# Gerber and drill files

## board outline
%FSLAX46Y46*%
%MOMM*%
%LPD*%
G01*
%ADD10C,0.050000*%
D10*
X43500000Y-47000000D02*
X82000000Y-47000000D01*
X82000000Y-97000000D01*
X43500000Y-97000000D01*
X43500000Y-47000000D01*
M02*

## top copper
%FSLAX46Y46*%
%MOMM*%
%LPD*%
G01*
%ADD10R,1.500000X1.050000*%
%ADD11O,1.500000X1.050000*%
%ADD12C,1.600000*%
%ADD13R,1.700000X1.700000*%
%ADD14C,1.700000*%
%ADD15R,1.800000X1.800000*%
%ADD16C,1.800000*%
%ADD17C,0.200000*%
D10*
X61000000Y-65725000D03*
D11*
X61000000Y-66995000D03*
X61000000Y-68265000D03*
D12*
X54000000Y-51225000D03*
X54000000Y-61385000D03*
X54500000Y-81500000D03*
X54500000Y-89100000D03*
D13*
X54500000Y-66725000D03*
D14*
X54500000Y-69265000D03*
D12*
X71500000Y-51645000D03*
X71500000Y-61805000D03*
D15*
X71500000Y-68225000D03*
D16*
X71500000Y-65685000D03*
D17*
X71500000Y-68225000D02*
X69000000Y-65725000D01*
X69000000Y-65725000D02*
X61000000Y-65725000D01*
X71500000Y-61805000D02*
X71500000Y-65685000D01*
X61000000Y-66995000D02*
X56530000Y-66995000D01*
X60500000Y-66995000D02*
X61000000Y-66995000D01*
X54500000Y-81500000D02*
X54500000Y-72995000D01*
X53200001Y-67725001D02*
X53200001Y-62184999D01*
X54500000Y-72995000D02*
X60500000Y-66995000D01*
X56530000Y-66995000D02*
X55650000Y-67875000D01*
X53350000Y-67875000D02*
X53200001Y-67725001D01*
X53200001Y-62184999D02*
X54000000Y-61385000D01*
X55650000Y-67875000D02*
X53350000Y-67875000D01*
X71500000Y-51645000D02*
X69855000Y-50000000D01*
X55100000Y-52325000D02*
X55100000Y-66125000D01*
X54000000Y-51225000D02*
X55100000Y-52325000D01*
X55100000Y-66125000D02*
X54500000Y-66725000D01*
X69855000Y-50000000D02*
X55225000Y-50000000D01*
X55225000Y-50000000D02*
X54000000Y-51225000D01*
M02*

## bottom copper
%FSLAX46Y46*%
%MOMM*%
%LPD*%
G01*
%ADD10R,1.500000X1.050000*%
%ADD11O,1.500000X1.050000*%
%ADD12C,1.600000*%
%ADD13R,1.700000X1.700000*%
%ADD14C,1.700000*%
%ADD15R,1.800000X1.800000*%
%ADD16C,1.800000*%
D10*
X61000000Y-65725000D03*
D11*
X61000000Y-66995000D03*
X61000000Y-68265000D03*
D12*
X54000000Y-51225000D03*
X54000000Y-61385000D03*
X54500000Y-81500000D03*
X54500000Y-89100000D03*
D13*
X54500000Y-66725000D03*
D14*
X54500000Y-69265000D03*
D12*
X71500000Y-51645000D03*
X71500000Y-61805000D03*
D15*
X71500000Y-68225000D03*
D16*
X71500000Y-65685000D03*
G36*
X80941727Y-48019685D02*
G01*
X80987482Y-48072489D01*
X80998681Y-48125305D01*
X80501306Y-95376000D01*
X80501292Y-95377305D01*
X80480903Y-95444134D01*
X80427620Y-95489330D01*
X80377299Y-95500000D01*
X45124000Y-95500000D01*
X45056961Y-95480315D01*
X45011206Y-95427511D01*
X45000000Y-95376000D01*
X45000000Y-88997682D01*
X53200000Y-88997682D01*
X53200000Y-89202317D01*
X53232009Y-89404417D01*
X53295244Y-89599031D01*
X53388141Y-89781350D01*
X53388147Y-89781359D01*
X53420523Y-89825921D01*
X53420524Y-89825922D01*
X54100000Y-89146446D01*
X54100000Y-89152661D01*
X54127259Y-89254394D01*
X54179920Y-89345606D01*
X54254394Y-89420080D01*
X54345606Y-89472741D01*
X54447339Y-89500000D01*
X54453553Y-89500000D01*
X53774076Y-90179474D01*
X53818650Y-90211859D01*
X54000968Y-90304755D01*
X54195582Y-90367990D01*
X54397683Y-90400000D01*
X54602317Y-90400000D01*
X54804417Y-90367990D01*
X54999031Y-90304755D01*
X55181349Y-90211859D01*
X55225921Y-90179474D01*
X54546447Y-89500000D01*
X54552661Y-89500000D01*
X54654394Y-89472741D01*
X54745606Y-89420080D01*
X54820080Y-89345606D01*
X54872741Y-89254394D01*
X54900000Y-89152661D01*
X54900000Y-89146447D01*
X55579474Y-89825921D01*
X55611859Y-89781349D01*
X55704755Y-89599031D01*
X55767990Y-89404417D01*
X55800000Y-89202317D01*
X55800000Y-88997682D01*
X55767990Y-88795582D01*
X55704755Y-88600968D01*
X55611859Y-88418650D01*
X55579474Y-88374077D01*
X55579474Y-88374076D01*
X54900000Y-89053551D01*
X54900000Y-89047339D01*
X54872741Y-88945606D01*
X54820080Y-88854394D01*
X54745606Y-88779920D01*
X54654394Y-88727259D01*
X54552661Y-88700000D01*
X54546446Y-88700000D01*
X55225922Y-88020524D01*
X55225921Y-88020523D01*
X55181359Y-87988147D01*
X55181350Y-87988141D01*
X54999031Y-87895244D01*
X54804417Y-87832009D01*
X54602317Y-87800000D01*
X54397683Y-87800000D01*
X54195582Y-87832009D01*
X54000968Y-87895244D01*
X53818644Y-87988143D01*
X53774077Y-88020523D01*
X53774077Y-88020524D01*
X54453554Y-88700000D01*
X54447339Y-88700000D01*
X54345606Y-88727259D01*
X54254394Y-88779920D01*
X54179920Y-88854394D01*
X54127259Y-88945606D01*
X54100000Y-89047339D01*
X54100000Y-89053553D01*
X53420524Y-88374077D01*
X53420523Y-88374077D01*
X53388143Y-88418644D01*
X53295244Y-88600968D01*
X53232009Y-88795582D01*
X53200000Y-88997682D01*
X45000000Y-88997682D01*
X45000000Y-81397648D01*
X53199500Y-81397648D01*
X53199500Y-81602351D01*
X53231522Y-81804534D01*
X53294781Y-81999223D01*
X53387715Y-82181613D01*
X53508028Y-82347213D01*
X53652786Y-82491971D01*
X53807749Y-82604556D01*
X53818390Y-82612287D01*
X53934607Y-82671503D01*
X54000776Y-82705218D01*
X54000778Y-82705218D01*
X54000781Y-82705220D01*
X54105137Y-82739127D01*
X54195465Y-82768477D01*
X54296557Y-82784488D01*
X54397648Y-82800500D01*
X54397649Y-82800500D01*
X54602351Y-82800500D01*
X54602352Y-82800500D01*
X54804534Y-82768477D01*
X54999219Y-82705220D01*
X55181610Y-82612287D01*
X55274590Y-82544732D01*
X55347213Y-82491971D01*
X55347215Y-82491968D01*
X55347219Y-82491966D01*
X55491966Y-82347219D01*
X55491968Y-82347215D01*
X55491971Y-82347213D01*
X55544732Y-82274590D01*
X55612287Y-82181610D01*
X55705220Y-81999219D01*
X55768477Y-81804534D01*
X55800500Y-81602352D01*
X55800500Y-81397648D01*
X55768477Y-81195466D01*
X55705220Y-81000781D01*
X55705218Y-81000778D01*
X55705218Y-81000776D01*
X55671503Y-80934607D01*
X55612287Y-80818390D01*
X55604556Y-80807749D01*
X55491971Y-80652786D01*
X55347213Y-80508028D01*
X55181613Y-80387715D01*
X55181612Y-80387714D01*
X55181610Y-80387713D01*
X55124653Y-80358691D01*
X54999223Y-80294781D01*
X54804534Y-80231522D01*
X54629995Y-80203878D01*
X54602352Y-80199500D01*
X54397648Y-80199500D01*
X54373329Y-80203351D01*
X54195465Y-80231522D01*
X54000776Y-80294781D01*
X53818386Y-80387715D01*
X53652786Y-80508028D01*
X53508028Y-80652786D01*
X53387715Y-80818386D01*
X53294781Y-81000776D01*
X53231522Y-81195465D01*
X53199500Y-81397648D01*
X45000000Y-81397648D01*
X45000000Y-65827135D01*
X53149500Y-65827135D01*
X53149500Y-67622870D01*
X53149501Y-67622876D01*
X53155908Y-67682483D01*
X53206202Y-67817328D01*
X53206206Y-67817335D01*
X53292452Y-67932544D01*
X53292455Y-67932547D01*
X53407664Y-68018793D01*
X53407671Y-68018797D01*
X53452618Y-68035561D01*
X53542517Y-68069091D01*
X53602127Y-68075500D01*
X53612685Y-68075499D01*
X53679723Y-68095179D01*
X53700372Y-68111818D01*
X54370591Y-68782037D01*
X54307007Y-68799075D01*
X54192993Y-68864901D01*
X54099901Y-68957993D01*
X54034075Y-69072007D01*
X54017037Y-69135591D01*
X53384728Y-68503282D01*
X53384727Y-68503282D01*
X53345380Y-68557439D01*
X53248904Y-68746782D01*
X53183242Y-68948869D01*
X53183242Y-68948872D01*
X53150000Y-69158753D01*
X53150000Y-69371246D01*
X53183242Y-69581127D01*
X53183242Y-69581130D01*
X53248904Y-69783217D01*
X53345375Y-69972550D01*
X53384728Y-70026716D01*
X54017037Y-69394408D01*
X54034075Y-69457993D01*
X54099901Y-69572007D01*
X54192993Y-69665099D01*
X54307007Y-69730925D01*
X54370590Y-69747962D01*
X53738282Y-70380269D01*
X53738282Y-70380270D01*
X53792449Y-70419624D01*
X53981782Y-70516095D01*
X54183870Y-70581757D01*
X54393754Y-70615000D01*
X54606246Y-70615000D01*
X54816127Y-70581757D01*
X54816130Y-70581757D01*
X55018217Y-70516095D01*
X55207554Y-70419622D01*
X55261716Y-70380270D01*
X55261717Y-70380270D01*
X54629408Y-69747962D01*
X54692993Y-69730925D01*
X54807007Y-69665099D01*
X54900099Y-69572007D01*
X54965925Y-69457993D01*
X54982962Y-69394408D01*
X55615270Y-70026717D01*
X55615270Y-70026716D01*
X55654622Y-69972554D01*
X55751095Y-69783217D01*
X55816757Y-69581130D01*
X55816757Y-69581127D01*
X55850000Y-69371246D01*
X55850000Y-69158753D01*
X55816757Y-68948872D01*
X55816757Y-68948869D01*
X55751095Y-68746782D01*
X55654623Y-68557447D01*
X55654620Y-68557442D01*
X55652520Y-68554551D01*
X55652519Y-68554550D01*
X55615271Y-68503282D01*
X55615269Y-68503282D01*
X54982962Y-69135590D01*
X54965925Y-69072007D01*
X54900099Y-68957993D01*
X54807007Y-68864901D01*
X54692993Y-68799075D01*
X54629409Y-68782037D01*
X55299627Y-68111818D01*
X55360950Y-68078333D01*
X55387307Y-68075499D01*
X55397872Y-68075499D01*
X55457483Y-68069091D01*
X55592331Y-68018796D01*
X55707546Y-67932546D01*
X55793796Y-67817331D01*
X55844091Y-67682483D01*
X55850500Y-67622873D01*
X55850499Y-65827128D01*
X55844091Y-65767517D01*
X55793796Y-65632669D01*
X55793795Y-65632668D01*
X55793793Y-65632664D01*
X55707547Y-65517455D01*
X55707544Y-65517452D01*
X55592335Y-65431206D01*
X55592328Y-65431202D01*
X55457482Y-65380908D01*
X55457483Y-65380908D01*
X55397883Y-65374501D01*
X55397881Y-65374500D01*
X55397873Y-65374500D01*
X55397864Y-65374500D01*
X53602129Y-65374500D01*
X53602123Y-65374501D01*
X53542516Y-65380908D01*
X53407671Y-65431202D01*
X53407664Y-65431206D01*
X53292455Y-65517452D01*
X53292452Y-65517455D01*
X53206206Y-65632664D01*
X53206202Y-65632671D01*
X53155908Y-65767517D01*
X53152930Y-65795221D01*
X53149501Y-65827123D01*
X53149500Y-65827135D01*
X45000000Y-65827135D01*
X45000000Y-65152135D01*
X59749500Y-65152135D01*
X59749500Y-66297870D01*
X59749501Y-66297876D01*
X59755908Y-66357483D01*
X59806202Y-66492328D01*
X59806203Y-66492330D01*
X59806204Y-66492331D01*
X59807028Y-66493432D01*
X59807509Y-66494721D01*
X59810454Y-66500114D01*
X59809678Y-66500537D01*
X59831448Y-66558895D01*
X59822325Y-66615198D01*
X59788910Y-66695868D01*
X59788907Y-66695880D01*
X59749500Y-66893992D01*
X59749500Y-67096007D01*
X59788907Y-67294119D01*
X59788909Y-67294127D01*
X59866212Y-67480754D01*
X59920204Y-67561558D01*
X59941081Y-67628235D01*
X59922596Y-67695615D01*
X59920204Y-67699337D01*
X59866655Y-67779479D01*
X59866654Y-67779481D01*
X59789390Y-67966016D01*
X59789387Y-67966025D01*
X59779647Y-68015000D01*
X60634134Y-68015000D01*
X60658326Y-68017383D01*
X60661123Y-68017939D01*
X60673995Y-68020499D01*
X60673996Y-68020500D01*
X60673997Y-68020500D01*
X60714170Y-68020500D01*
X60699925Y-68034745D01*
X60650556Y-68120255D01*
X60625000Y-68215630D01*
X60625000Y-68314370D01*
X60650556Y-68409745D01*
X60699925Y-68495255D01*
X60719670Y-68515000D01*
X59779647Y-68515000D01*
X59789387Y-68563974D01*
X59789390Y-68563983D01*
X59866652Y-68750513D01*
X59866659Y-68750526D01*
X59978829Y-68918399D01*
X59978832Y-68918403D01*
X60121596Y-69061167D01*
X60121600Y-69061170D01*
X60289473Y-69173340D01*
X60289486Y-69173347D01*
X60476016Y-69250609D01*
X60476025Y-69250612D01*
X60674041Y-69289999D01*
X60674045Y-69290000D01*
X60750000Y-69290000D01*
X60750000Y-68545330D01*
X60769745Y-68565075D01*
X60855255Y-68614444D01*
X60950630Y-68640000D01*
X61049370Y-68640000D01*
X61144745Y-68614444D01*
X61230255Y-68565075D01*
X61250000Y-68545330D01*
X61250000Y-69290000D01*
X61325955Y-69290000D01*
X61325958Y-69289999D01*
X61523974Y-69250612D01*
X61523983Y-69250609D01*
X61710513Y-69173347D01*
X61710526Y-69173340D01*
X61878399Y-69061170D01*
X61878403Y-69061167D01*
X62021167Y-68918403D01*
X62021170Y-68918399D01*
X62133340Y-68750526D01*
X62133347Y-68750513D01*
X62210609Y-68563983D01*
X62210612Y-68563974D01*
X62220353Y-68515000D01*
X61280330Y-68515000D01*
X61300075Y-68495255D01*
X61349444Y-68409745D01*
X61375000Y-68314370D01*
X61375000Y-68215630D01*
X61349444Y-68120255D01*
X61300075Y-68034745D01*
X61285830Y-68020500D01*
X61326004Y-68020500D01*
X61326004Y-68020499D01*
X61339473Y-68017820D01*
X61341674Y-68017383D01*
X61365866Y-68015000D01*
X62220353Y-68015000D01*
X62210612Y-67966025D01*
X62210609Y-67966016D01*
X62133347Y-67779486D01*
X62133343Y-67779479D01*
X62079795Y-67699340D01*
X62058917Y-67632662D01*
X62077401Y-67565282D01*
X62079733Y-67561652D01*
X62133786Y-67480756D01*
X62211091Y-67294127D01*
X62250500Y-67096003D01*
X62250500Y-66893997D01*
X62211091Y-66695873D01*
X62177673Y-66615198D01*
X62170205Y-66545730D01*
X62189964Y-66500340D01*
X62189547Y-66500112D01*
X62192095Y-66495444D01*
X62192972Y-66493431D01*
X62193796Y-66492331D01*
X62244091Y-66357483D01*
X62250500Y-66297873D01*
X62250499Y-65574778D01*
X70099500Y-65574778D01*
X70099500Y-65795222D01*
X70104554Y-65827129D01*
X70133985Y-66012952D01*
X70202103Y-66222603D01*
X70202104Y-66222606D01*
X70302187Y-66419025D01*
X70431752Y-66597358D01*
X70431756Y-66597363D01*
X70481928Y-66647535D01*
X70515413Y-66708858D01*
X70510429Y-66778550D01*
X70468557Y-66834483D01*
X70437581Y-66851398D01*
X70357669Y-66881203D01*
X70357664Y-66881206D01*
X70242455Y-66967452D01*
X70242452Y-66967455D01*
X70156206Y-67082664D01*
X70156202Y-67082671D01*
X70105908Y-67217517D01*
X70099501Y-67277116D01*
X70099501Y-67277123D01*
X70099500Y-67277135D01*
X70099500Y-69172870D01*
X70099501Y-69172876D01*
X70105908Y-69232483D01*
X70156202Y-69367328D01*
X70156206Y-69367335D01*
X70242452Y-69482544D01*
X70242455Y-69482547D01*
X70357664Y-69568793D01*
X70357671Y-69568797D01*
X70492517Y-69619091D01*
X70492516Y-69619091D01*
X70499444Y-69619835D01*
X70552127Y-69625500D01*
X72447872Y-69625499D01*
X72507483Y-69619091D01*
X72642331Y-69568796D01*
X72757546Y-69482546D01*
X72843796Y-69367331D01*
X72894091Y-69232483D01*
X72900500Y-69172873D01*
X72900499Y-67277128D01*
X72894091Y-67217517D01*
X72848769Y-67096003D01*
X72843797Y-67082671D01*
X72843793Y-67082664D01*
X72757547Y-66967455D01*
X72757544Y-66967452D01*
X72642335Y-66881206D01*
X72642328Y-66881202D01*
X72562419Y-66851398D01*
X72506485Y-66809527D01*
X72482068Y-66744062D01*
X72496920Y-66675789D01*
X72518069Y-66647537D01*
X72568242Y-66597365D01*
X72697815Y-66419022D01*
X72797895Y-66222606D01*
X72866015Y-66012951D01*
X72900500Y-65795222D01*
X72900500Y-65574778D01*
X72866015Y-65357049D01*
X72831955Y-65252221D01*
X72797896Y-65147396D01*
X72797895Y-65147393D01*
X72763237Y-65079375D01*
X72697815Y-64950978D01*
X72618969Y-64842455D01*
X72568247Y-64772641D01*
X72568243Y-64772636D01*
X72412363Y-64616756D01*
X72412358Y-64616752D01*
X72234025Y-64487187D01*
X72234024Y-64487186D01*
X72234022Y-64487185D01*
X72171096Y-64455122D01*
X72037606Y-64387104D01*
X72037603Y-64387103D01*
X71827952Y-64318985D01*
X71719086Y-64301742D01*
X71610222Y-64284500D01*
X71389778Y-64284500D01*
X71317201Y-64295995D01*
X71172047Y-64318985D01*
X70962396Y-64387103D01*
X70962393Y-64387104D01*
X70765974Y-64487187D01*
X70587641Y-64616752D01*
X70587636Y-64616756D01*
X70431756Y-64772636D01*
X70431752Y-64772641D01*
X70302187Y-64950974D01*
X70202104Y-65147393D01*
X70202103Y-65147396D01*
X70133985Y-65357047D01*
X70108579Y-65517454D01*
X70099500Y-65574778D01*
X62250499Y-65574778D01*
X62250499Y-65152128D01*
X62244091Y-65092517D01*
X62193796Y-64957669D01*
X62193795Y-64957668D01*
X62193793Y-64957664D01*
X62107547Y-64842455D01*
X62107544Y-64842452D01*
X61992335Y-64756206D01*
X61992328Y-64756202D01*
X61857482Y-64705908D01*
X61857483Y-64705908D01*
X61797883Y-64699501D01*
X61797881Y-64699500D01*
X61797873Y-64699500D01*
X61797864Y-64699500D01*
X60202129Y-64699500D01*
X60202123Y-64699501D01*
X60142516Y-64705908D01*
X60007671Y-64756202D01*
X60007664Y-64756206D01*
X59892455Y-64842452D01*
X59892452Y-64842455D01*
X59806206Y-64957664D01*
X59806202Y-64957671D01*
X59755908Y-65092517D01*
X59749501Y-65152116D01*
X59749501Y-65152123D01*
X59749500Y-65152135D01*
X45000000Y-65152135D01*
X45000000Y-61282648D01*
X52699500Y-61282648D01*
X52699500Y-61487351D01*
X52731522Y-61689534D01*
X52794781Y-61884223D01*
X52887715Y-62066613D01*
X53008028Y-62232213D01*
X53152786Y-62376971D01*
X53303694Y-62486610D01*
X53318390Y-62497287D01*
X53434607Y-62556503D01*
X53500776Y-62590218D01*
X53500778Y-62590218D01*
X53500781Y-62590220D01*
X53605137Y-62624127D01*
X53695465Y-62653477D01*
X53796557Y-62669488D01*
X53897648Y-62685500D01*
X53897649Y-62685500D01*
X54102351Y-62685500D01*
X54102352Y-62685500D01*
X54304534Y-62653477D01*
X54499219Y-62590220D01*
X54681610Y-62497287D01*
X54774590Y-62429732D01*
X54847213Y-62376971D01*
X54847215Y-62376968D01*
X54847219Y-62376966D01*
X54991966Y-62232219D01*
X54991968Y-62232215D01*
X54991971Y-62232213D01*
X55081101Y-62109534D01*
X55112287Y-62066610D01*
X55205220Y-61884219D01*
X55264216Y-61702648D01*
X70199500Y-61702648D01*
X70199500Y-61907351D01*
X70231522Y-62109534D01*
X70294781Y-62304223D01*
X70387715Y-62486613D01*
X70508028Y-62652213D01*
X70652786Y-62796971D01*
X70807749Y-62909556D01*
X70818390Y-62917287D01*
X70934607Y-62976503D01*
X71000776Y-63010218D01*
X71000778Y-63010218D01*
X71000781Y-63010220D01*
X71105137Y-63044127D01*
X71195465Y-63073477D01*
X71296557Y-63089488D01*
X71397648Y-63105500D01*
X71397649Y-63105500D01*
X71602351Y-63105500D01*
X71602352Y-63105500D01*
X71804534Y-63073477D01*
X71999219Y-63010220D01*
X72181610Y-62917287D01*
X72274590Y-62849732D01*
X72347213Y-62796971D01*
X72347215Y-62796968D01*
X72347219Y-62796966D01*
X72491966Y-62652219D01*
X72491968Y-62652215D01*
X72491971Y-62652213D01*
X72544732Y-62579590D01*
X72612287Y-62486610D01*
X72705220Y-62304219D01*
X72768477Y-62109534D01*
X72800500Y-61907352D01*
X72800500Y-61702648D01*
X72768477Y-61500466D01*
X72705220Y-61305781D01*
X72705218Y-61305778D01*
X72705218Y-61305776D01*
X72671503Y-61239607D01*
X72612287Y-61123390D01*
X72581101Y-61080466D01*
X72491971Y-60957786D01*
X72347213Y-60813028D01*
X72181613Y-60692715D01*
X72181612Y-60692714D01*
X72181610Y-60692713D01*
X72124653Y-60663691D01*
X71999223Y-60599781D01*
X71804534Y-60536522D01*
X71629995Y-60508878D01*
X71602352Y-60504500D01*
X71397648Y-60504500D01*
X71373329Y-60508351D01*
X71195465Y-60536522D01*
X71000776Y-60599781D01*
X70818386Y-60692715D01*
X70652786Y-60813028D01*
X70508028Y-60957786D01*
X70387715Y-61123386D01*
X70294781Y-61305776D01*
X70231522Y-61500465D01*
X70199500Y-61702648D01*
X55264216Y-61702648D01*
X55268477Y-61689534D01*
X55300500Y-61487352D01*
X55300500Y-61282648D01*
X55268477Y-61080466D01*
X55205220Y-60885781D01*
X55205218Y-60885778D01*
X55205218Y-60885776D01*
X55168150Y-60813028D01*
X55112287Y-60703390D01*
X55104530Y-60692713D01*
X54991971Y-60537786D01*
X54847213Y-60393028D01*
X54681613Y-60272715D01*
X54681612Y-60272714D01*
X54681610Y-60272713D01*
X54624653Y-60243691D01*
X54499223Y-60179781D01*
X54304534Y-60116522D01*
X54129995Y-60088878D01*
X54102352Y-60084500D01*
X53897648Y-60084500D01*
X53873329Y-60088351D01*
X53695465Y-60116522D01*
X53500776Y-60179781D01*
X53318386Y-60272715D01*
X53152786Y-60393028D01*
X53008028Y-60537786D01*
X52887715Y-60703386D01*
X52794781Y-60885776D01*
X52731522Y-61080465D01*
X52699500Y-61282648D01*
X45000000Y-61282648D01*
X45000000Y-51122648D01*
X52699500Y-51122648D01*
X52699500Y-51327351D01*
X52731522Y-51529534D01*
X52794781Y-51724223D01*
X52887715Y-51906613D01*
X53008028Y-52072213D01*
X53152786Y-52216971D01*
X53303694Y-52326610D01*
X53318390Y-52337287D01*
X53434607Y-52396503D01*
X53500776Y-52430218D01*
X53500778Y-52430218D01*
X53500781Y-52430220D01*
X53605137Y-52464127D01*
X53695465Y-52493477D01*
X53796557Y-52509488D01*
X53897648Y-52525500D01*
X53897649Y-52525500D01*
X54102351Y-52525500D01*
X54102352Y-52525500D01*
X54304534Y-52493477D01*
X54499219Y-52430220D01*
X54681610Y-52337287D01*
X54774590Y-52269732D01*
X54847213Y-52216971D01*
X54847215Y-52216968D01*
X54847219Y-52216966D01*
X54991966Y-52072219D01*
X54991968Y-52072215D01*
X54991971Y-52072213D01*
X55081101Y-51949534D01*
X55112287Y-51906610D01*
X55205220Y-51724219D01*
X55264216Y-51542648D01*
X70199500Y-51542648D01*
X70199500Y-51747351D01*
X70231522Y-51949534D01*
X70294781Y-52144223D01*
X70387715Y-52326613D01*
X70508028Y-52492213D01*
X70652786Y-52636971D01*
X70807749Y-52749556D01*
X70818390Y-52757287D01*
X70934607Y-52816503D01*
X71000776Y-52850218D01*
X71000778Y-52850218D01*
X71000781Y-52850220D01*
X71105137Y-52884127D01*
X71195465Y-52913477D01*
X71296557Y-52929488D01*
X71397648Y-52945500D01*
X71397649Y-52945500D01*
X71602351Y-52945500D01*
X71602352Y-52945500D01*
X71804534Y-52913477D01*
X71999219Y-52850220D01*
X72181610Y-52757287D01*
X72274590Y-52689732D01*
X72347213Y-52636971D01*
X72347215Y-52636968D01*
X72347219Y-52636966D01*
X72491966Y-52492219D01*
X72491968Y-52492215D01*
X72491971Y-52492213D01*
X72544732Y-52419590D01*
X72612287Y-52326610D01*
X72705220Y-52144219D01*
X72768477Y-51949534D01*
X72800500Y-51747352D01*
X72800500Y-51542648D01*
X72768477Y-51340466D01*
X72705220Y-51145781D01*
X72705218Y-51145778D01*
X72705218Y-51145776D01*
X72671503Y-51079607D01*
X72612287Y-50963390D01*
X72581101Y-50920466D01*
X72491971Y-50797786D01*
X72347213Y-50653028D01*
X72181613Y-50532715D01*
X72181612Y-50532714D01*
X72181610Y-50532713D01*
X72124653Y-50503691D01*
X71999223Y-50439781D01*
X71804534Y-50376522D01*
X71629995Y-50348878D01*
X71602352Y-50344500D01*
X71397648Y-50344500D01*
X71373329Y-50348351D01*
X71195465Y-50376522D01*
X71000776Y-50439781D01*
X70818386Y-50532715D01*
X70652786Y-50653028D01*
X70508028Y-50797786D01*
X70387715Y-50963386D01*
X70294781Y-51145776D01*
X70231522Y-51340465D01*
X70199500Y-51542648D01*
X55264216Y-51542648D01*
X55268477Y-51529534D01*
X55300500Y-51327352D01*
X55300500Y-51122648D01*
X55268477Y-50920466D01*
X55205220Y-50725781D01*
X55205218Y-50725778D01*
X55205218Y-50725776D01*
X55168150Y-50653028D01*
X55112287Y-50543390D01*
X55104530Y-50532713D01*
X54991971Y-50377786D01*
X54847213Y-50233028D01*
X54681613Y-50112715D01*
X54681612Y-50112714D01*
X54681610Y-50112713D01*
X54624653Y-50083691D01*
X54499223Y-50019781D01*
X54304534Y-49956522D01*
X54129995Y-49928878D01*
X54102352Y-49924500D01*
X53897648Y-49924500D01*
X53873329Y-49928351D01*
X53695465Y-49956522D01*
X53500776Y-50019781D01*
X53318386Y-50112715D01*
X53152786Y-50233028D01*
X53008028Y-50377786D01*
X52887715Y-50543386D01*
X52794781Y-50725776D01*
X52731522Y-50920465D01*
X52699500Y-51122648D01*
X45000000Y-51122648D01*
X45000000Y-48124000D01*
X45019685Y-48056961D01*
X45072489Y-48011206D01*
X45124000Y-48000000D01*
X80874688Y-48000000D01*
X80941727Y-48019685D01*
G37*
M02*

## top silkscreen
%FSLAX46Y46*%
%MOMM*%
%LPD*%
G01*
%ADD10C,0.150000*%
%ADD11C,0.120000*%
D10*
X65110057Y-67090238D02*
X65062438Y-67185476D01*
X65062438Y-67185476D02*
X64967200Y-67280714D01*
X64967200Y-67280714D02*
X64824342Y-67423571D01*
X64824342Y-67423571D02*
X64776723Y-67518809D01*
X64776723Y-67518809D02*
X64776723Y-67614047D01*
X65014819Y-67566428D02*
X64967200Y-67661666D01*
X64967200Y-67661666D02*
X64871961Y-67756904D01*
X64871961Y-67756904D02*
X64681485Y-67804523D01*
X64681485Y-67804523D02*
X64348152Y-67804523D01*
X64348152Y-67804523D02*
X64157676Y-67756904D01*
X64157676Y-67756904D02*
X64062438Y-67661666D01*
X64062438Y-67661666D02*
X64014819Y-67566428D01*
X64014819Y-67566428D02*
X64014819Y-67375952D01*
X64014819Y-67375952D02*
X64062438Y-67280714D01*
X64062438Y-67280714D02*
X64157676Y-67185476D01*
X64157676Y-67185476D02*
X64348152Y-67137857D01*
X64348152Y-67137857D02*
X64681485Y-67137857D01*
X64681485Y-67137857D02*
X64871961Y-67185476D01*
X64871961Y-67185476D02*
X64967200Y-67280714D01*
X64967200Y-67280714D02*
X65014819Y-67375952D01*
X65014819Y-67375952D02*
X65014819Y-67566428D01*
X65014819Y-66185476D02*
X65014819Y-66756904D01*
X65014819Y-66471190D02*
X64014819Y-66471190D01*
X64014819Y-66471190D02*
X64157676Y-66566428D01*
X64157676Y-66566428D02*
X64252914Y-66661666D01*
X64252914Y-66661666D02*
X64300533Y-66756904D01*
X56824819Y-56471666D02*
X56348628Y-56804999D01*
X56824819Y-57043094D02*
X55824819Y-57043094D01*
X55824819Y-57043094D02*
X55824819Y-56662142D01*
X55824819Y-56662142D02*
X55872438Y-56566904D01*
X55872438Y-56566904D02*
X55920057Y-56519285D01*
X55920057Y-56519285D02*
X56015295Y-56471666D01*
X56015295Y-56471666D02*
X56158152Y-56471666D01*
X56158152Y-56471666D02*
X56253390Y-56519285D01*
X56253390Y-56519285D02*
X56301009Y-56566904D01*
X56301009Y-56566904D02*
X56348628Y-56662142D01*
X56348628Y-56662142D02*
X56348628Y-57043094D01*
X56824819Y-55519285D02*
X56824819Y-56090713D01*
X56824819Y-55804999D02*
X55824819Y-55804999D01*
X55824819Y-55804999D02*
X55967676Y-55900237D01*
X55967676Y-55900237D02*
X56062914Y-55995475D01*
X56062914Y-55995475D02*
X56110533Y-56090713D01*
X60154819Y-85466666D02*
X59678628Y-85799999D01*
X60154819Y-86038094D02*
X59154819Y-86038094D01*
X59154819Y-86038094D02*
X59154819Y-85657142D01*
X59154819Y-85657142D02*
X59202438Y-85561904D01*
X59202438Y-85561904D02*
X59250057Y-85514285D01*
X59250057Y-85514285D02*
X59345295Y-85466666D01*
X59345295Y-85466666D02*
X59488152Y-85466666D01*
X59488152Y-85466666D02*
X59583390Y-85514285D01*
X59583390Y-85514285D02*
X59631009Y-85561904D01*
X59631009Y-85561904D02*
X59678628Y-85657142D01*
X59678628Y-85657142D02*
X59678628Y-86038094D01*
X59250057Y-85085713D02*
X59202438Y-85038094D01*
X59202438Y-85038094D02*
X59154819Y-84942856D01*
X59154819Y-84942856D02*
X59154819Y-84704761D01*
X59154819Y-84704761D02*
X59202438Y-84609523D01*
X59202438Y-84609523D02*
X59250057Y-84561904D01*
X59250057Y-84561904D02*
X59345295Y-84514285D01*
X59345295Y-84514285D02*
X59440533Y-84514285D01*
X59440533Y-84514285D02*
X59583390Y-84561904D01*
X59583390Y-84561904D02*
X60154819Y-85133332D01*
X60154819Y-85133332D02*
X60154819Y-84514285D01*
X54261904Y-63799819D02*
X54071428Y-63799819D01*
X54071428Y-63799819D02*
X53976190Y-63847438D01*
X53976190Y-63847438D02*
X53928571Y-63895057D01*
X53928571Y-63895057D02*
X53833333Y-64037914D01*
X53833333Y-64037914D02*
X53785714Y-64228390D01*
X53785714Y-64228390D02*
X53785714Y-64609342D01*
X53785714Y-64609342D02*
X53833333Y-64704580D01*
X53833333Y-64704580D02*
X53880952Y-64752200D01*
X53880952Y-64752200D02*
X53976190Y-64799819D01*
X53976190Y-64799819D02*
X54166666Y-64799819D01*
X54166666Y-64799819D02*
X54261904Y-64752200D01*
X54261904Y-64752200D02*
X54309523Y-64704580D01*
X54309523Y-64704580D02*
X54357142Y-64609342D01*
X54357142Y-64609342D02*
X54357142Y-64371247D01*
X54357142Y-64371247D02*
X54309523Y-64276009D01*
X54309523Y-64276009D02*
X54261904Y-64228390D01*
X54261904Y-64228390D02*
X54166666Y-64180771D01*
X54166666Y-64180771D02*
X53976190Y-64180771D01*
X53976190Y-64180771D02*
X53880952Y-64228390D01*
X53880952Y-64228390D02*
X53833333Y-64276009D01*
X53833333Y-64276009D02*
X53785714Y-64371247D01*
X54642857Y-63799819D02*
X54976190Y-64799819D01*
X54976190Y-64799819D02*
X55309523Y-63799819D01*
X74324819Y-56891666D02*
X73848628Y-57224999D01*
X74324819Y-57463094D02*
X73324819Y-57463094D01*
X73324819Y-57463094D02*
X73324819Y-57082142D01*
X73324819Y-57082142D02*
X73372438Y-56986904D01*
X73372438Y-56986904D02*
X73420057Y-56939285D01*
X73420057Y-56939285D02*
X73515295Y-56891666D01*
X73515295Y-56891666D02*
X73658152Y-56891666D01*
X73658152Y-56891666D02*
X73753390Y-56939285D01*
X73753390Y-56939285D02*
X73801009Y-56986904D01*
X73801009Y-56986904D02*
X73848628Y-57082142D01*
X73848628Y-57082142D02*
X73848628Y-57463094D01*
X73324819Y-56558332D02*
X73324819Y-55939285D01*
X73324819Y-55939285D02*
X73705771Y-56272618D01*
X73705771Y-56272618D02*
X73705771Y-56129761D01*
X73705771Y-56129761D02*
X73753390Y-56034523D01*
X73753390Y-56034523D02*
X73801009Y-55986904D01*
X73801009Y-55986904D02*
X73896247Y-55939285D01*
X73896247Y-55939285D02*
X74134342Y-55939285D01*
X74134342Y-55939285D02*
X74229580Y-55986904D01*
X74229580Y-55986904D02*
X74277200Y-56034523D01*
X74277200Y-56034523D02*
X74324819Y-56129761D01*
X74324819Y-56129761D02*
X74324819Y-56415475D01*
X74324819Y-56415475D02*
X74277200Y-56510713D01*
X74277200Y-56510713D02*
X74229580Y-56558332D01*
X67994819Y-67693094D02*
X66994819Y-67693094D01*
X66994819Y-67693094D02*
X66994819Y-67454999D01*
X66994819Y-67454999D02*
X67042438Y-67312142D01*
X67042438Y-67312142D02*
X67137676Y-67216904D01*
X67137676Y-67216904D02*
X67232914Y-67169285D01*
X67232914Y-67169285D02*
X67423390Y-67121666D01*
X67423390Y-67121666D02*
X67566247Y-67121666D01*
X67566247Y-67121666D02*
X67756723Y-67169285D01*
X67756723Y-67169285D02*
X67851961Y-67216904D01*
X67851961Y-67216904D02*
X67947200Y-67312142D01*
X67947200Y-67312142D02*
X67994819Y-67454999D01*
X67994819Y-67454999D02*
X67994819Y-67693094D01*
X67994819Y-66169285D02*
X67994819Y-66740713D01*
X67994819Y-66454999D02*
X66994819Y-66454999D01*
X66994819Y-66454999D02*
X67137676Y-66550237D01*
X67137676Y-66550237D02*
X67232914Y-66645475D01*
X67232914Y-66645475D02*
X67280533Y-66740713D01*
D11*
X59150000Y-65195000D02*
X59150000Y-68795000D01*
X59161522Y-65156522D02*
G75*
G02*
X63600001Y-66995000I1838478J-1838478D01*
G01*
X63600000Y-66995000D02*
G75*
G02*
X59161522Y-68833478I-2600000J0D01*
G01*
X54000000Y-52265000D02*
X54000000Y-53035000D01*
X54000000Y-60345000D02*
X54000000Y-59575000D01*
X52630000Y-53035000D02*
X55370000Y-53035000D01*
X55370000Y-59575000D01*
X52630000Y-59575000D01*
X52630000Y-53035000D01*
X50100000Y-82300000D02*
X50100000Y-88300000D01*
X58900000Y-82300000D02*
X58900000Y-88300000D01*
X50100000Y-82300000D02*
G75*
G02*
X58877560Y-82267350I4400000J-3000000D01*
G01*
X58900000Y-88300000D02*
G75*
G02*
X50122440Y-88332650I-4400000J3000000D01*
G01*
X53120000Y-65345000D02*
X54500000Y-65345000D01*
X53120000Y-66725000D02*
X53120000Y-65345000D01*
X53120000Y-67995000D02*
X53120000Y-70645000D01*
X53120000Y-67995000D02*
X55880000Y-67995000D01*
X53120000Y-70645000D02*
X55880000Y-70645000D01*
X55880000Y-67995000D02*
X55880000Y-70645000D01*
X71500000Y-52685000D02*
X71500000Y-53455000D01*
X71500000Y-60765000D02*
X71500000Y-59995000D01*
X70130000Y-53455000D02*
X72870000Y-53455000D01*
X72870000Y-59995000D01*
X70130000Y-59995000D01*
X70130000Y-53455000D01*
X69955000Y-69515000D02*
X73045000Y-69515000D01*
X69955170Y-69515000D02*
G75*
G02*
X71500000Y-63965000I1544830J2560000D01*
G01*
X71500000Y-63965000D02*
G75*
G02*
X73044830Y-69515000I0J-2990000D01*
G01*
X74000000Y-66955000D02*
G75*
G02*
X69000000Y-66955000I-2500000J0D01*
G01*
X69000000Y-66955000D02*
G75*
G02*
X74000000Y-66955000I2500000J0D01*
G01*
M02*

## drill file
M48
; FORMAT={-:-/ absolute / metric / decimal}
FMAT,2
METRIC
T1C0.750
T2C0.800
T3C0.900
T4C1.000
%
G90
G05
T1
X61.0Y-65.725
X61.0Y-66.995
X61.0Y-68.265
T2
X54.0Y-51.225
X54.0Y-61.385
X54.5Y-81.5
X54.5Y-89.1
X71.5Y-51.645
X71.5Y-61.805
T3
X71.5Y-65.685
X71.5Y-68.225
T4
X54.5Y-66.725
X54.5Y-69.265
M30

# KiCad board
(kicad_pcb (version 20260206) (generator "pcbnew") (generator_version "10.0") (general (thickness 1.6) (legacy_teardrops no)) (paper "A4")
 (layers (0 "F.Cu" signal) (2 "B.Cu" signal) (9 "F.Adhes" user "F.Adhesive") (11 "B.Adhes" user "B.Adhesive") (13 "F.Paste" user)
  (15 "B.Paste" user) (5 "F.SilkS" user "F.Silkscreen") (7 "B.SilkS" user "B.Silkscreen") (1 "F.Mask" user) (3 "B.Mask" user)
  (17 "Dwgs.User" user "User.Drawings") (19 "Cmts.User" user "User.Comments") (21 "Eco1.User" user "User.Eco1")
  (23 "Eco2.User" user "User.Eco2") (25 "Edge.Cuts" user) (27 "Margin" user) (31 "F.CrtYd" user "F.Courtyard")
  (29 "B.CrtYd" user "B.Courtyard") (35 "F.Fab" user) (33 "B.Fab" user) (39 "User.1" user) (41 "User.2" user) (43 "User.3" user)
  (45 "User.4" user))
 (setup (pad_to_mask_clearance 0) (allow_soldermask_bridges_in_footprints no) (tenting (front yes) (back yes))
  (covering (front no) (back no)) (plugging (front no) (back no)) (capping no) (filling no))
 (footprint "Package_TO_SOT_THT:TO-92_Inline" (layer "F.Cu") (at 61 65.725 -90)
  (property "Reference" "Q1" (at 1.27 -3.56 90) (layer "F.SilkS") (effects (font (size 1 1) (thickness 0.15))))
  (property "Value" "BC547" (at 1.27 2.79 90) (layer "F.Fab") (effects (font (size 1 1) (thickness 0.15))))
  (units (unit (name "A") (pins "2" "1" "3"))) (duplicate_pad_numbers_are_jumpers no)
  (fp_line (start -0.53 1.85) (end 3.07 1.85) (stroke (width 0.12) (type solid)) (layer "F.SilkS"))
  (fp_arc (start -0.568478 1.838478) (mid -1.132087 -0.994977) (end 1.27 -2.6) (stroke (width 0.12) (type solid)) (layer "F.SilkS"))
  (fp_arc (start 1.27 -2.6) (mid 3.672087 -0.994977) (end 3.108478 1.838478) (stroke (width 0.12) (type solid)) (layer "F.SilkS"))
  (pad "1" thru_hole rect (at 0 0 270) (size 1.05 1.5) (drill 0.75) (layers "*.Cu" "*.Mask") (remove_unused_layers no) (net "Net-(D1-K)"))
  (pad "2" thru_hole oval (at 1.27 0 270) (size 1.05 1.5) (drill 0.75) (layers "*.Cu" "*.Mask") (remove_unused_layers no) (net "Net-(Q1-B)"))
  (pad "3" thru_hole oval (at 2.54 0 270) (size 1.05 1.5) (drill 0.75) (layers "*.Cu" "*.Mask") (remove_unused_layers no) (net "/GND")))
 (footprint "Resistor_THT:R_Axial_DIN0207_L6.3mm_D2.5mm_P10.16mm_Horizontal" (layer "F.Cu") (at 54 51.225 -90)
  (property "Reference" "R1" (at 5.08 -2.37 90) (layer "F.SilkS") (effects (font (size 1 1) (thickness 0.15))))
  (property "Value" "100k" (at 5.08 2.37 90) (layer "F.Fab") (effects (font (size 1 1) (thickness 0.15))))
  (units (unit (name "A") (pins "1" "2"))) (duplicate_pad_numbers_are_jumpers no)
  (fp_line (start 1.04 0) (end 1.81 0) (stroke (width 0.12) (type solid)) (layer "F.SilkS"))
  (fp_line (start 9.12 0) (end 8.35 0) (stroke (width 0.12) (type solid)) (layer "F.SilkS"))
  (fp_rect (start 1.81 -1.37) (end 8.35 1.37) (stroke (width 0.12) (type solid)) (fill no) (layer "F.SilkS"))
  (pad "1" thru_hole circle (at 0 0 270) (size 1.6 1.6) (drill 0.8) (layers "*.Cu" "*.Mask") (remove_unused_layers no) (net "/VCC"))
  (pad "2" thru_hole circle (at 10.16 0 270) (size 1.6 1.6) (drill 0.8) (layers "*.Cu" "*.Mask") (remove_unused_layers no)
   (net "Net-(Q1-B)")))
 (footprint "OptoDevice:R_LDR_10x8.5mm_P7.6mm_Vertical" (layer "F.Cu") (at 54.5 81.5 -90)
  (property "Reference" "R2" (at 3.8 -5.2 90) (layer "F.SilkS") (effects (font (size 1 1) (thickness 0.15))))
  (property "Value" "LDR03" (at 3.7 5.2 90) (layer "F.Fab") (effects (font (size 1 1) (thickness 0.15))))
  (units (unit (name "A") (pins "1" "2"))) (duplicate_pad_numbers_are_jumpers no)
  (fp_line (start 0.8 4.4) (end 6.8 4.4) (stroke (width 0.12) (type solid)) (layer "F.SilkS"))
  (fp_line (start 0.8 -4.4) (end 6.8 -4.4) (stroke (width 0.12) (type solid)) (layer "F.SilkS"))
  (fp_arc (start 0.8 4.4) (mid -1.525374 0.019809) (end 0.76735 -4.37756) (stroke (width 0.12) (type solid)) (layer "F.SilkS"))
  (fp_arc (start 6.8 -4.4) (mid 9.125374 -0.019809) (end 6.83265 4.37756) (stroke (width 0.12) (type solid)) (layer "F.SilkS"))
  (pad "1" thru_hole circle (at 0 0 270) (size 1.6 1.6) (drill 0.8) (layers "*.Cu" "*.Mask") (remove_unused_layers no) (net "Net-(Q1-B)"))
  (pad "2" thru_hole circle (at 7.6 0 270) (size 1.6 1.6) (drill 0.8) (layers "*.Cu" "*.Mask") (remove_unused_layers no) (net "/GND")))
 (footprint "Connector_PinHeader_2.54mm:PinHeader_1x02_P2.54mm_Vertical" (layer "F.Cu") (at 54.5 66.725)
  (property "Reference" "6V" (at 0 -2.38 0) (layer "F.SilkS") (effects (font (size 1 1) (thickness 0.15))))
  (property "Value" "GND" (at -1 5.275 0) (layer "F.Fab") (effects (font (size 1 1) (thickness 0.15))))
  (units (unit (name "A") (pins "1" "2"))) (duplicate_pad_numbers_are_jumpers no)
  (fp_line (start -1.38 -1.38) (end 0 -1.38) (stroke (width 0.12) (type solid)) (layer "F.SilkS"))
  (fp_line (start -1.38 0) (end -1.38 -1.38) (stroke (width 0.12) (type solid)) (layer "F.SilkS"))
  (fp_line (start -1.38 1.27) (end -1.38 3.92) (stroke (width 0.12) (type solid)) (layer "F.SilkS"))
  (fp_line (start -1.38 1.27) (end 1.38 1.27) (stroke (width 0.12) (type solid)) (layer "F.SilkS"))
  (fp_line (start -1.38 3.92) (end 1.38 3.92) (stroke (width 0.12) (type solid)) (layer "F.SilkS"))
  (fp_line (start 1.38 1.27) (end 1.38 3.92) (stroke (width 0.12) (type solid)) (layer "F.SilkS"))
  (pad "1" thru_hole rect (at 0 0) (size 1.7 1.7) (drill 1) (layers "*.Cu" "*.Mask") (remove_unused_layers no) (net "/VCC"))
  (pad "2" thru_hole circle (at 0 2.54) (size 1.7 1.7) (drill 1) (layers "*.Cu" "*.Mask") (remove_unused_layers no) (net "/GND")))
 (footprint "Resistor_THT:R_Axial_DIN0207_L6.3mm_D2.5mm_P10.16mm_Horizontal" (layer "F.Cu") (at 71.5 51.645 -90)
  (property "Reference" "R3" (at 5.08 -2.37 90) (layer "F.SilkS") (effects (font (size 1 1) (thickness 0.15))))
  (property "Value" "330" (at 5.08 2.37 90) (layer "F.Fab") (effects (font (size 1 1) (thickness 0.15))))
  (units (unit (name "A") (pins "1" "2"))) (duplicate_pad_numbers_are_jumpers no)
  (fp_line (start 1.04 0) (end 1.81 0) (stroke (width 0.12) (type solid)) (layer "F.SilkS"))
  (fp_line (start 9.12 0) (end 8.35 0) (stroke (width 0.12) (type solid)) (layer "F.SilkS"))
  (fp_rect (start 1.81 -1.37) (end 8.35 1.37) (stroke (width 0.12) (type solid)) (fill no) (layer "F.SilkS"))
  (pad "1" thru_hole circle (at 0 0 270) (size 1.6 1.6) (drill 0.8) (layers "*.Cu" "*.Mask") (remove_unused_layers no) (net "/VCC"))
  (pad "2" thru_hole circle (at 10.16 0 270) (size 1.6 1.6) (drill 0.8) (layers "*.Cu" "*.Mask") (remove_unused_layers no)
   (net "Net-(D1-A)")))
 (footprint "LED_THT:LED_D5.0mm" (layer "F.Cu") (at 71.5 68.225 90)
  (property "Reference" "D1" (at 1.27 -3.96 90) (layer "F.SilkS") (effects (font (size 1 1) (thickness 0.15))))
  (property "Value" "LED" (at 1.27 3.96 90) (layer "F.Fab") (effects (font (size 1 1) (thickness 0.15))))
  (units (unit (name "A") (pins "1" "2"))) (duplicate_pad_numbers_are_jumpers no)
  (fp_line (start -1.29 -1.545) (end -1.29 1.545) (stroke (width 0.12) (type solid)) (layer "F.SilkS"))
  (fp_arc (start -1.29 -1.54483) (mid 2.071779 -2.880495) (end 4.26 0) (stroke (width 0.12) (type solid)) (layer "F.SilkS"))
  (fp_arc (start 4.26 0) (mid 2.071779 2.880495) (end -1.29 1.54483) (stroke (width 0.12) (type solid)) (layer "F.SilkS"))
  (fp_circle (center 1.27 0) (end 3.77 0) (stroke (width 0.12) (type solid)) (fill no) (layer "F.SilkS"))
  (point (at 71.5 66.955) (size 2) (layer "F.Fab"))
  (pad "1" thru_hole rect (at 0 0 90) (size 1.8 1.8) (drill 0.9) (layers "*.Cu" "*.Mask") (remove_unused_layers no) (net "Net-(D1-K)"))
  (pad "2" thru_hole circle (at 2.54 0 90) (size 1.8 1.8) (drill 0.9) (layers "*.Cu" "*.Mask") (remove_unused_layers no) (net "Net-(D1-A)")))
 (gr_rect (start 43.5 47) (end 82 97) (stroke (width 0.05) (type default)) (fill no) (layer "Edge.Cuts"))
 (segment (start 71.5 68.225) (end 69 65.725) (width 0.2) (layer "F.Cu") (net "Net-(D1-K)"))
 (segment (start 69 65.725) (end 61 65.725) (width 0.2) (layer "F.Cu") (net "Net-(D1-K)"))
 (segment (start 71.5 61.805) (end 71.5 65.685) (width 0.2) (layer "F.Cu") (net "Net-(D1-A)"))
 (segment (start 61 66.995) (end 56.53 66.995) (width 0.2) (layer "F.Cu") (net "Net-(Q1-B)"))
 (segment (start 60.5 66.995) (end 61 66.995) (width 0.2) (layer "F.Cu") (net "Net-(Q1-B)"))
 (segment (start 54.5 81.5) (end 54.5 72.995) (width 0.2) (layer "F.Cu") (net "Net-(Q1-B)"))
 (segment (start 53.200001 67.725001) (end 53.200001 62.184999) (width 0.2) (layer "F.Cu") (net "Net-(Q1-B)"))
 (segment (start 54.5 72.995) (end 60.5 66.995) (width 0.2) (layer "F.Cu") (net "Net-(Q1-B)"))
 (segment (start 56.53 66.995) (end 55.65 67.875) (width 0.2) (layer "F.Cu") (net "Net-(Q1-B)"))
 (segment (start 53.35 67.875) (end 53.200001 67.725001) (width 0.2) (layer "F.Cu") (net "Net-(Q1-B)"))
 (segment (start 53.200001 62.184999) (end 54 61.385) (width 0.2) (layer "F.Cu") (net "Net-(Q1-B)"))
 (segment (start 55.65 67.875) (end 53.35 67.875) (width 0.2) (layer "F.Cu") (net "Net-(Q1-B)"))
 (segment (start 71.5 51.645) (end 69.855 50) (width 0.2) (layer "F.Cu") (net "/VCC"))
 (segment (start 55.1 52.325) (end 55.1 66.125) (width 0.2) (layer "F.Cu") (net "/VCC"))
 (segment (start 54 51.225) (end 55.1 52.325) (width 0.2) (layer "F.Cu") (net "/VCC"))
 (segment (start 55.1 66.125) (end 54.5 66.725) (width 0.2) (layer "F.Cu") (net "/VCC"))
 (segment (start 69.855 50) (end 55.225 50) (width 0.2) (layer "F.Cu") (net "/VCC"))
 (segment (start 55.225 50) (end 54 51.225) (width 0.2) (layer "F.Cu") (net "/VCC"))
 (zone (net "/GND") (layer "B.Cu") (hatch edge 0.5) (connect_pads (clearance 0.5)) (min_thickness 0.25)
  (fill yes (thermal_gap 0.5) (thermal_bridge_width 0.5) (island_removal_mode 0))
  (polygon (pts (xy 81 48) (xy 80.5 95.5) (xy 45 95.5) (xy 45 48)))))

